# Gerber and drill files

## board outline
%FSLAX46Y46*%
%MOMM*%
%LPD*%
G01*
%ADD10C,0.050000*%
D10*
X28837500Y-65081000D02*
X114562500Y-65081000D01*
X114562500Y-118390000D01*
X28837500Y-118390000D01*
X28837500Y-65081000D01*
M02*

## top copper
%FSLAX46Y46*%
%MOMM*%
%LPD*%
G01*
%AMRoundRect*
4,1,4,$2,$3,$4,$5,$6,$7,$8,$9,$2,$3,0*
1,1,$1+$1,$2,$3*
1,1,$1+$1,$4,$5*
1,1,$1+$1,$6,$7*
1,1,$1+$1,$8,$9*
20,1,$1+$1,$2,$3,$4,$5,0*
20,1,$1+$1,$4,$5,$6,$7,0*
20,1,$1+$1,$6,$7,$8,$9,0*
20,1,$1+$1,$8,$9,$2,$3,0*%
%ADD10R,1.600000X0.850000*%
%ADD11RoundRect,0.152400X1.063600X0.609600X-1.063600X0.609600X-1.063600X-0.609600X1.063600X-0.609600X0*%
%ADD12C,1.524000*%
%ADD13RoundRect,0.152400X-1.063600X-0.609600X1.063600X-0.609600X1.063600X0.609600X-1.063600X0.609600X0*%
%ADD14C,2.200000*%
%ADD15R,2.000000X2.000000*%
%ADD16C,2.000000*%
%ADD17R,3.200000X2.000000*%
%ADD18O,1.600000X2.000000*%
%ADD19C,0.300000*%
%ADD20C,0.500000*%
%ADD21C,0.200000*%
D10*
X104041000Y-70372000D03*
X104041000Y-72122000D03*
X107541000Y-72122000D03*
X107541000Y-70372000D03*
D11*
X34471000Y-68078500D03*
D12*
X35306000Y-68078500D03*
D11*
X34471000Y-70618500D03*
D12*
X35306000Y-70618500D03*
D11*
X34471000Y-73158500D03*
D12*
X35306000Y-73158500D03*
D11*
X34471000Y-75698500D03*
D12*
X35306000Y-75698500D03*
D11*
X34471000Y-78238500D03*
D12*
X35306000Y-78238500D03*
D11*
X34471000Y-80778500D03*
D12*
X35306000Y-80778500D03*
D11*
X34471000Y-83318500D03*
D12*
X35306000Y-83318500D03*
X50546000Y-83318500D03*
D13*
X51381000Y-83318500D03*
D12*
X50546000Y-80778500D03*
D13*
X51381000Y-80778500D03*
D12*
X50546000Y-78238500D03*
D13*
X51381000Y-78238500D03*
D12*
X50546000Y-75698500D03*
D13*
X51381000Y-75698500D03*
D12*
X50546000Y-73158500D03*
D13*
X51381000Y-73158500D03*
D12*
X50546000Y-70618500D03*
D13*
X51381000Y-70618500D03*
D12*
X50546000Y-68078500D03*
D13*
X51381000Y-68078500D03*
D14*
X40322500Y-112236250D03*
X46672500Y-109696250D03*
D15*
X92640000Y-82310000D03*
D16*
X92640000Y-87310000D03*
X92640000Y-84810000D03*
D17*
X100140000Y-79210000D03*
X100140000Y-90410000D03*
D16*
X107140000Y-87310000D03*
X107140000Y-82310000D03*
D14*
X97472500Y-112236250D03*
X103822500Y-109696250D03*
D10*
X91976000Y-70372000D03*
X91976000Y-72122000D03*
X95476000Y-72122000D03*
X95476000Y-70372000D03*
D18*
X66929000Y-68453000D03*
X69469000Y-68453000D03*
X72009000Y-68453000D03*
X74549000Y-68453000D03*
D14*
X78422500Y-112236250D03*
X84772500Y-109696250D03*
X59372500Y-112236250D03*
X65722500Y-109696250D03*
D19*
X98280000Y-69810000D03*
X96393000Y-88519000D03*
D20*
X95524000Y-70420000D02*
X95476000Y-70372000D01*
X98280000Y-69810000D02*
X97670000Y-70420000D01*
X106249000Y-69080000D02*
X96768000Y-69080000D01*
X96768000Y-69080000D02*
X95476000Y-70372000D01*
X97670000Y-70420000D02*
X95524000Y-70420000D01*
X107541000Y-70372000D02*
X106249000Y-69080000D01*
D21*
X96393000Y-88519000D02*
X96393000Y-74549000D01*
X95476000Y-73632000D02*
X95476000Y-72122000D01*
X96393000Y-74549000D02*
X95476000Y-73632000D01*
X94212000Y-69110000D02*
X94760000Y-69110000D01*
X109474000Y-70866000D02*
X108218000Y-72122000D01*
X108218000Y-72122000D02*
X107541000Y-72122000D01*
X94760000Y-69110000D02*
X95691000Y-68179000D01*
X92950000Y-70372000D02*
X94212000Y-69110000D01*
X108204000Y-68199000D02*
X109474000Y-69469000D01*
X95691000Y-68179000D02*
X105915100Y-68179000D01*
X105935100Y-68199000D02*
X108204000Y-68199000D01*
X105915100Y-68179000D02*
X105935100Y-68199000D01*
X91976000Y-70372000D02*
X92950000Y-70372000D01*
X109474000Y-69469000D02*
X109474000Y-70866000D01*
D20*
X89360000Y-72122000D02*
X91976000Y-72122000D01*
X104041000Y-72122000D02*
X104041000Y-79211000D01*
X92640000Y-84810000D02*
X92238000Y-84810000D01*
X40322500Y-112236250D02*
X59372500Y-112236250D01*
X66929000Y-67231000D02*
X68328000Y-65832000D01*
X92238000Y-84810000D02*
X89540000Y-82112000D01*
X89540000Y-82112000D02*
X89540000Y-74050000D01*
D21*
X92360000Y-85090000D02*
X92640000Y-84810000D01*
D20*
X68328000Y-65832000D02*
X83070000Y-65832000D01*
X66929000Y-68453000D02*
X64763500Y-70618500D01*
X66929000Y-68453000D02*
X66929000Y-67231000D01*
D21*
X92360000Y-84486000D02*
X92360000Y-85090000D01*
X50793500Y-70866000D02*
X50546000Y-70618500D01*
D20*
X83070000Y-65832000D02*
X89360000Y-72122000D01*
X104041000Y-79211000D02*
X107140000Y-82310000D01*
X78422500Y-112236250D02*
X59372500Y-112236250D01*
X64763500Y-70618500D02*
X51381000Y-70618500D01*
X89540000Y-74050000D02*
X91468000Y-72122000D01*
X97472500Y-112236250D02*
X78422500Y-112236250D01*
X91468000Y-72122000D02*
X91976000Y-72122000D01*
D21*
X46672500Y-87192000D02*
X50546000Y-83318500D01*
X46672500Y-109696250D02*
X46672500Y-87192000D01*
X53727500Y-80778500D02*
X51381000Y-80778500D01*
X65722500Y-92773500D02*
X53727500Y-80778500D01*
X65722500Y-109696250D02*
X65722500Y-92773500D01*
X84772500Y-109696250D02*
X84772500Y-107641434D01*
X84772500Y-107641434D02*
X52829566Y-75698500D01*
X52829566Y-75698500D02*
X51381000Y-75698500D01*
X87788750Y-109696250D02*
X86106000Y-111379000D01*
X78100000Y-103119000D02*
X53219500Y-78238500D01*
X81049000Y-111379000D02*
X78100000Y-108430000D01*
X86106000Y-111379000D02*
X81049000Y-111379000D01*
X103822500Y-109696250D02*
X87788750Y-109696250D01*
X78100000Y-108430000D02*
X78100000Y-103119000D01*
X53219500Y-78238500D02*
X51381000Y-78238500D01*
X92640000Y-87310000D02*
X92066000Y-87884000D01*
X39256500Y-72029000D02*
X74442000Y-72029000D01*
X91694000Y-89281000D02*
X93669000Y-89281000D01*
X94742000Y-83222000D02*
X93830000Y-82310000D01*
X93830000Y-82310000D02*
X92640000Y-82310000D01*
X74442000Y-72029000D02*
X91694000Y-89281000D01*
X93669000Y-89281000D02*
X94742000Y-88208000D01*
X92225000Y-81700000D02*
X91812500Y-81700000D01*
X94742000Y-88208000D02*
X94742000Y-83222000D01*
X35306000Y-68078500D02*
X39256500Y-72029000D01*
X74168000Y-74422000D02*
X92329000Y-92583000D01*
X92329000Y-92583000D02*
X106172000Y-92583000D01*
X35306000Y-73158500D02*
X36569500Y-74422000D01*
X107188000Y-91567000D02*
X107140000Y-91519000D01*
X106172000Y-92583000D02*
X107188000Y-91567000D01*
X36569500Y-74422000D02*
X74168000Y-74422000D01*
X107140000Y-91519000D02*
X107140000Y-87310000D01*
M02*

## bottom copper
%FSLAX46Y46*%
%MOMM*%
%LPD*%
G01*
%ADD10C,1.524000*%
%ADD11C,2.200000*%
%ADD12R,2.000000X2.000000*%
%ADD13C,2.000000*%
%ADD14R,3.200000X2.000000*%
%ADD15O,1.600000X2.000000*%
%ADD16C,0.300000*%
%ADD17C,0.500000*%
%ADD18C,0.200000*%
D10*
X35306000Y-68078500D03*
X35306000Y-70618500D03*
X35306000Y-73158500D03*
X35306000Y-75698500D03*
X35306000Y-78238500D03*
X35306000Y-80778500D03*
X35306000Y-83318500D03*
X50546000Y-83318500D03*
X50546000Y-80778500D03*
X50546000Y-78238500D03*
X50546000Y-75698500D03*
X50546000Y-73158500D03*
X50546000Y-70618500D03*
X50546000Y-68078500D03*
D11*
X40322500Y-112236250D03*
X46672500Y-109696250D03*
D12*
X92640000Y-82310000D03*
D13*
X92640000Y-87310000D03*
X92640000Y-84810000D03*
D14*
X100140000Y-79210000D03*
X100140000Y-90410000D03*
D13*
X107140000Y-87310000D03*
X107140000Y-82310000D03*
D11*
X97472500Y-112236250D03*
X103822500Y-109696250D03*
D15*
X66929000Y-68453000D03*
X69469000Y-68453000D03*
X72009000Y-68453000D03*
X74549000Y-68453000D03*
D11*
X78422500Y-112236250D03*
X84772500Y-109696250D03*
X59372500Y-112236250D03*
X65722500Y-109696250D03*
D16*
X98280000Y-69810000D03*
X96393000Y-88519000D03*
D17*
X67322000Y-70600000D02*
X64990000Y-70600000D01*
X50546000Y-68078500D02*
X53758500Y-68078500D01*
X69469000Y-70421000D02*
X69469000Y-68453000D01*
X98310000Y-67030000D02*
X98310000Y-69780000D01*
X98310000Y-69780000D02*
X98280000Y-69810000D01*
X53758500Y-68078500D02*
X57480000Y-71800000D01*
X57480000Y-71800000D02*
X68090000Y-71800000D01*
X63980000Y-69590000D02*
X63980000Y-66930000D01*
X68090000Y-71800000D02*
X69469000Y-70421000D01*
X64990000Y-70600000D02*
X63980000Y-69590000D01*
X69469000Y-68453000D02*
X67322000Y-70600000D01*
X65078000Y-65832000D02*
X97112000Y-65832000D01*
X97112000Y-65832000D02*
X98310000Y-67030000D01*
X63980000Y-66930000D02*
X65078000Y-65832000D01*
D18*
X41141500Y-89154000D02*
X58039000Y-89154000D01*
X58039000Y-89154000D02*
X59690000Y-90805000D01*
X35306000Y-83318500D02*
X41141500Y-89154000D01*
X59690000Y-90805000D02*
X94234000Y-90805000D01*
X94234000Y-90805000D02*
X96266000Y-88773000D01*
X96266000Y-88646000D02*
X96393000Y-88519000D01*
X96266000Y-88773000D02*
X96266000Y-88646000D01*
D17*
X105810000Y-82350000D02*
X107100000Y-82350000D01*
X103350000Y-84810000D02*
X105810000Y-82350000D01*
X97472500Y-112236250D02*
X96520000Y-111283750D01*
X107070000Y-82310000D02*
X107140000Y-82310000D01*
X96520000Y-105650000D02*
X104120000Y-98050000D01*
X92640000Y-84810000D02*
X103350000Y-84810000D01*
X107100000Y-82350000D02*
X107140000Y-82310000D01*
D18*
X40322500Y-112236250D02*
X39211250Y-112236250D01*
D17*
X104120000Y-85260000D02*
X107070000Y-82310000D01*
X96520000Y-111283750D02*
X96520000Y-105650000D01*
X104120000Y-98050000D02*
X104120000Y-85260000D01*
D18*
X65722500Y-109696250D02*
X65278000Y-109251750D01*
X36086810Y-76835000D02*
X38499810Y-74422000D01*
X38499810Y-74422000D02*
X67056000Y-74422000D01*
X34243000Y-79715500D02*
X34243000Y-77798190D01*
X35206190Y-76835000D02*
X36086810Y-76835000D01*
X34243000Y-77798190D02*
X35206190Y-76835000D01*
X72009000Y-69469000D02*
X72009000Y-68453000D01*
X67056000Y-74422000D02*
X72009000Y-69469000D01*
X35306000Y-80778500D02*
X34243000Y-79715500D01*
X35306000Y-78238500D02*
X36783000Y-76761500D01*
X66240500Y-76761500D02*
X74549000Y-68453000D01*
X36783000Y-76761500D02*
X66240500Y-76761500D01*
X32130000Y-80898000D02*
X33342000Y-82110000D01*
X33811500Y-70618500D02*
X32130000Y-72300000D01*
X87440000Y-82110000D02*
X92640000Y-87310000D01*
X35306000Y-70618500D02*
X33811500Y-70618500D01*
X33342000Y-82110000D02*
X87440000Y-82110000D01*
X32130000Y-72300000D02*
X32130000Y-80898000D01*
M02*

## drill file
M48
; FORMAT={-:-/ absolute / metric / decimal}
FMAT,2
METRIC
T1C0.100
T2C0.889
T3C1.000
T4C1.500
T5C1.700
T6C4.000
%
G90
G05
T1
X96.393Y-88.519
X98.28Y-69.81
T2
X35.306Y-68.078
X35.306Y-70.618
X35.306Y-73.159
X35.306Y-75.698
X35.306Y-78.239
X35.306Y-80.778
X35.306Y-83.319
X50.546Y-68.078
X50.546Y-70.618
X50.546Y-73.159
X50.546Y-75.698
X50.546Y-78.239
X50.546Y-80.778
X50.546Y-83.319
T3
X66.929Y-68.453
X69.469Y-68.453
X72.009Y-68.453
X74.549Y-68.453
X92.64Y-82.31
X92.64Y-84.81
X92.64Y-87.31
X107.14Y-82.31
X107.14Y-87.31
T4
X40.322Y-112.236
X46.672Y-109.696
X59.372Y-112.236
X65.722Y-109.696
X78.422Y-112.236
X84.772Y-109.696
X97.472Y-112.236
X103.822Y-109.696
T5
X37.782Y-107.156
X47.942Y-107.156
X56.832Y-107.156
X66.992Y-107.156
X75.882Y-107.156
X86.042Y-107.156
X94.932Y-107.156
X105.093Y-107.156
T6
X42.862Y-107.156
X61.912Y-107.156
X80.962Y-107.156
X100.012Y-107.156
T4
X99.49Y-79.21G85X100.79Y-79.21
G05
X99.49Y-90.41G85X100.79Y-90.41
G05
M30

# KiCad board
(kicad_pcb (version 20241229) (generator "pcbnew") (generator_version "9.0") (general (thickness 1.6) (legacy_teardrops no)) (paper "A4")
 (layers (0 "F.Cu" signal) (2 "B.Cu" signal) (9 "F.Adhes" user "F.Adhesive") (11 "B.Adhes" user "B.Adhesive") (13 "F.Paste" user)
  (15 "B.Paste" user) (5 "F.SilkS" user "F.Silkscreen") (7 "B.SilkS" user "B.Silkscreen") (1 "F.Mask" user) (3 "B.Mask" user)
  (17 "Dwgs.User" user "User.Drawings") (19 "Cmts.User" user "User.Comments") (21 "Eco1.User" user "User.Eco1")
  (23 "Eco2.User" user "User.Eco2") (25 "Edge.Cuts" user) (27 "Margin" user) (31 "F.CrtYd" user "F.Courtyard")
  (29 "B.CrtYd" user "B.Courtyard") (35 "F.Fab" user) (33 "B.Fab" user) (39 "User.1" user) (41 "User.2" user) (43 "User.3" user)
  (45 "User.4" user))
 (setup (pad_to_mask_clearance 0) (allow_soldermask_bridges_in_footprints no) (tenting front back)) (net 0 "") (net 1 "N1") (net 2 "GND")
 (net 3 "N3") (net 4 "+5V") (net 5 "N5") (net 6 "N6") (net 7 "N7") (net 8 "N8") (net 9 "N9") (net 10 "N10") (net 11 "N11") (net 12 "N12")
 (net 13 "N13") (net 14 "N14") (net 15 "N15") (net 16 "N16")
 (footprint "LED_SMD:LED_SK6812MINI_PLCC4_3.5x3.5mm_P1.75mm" (layer "F.Cu") (at 105.791 71.247)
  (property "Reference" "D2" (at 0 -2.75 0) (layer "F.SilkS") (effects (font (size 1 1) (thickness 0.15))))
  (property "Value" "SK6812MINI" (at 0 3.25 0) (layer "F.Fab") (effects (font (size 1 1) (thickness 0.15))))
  (pad "1" smd rect (at -1.75 -0.875) (size 1.6 0.85) (layers "F.Cu" "F.Mask" "F.Paste") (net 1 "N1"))
  (pad "2" smd rect (at -1.75 0.875) (size 1.6 0.85) (layers "F.Cu" "F.Mask" "F.Paste") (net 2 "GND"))
  (pad "3" smd rect (at 1.75 0.875) (size 1.6 0.85) (layers "F.Cu" "F.Mask" "F.Paste") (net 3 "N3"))
  (pad "4" smd rect (at 1.75 -0.875) (size 1.6 0.85) (layers "F.Cu" "F.Mask" "F.Paste") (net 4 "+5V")))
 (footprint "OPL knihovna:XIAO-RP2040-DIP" (layer "F.Cu") (at 42.926 75.6985)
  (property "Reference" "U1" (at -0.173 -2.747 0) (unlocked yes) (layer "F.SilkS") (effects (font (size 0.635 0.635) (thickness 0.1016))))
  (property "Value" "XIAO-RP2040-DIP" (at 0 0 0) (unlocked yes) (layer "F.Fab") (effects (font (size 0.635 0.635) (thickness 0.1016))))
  (pad "1" smd roundrect (at -8.455 -7.62 180) (size 2.432 1.524) (layers "F.Cu" "F.Mask") (roundrect_rratio 0.1) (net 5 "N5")
   (thermal_bridge_angle 45))
  (pad "1" thru_hole circle (at -7.62 -7.62 180) (size 1.524 1.524) (drill 0.889) (layers "*.Cu" "*.Mask") (remove_unused_layers no)
   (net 5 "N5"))
  (pad "2" smd roundrect (at -8.455 -5.08 180) (size 2.432 1.524) (layers "F.Cu" "F.Mask") (roundrect_rratio 0.1) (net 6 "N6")
   (thermal_bridge_angle 45))
  (pad "2" thru_hole circle (at -7.62 -5.08 180) (size 1.524 1.524) (drill 0.889) (layers "*.Cu" "*.Mask") (remove_unused_layers no)
   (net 6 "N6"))
  (pad "3" smd roundrect (at -8.455 -2.54 180) (size 2.432 1.524) (layers "F.Cu" "F.Mask") (roundrect_rratio 0.1) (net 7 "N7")
   (thermal_bridge_angle 45))
  (pad "3" thru_hole circle (at -7.62 -2.54 180) (size 1.524 1.524) (drill 0.889) (layers "*.Cu" "*.Mask") (remove_unused_layers no)
   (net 7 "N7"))
  (pad "4" smd roundrect (at -8.455 0 180) (size 2.432 1.524) (layers "F.Cu" "F.Mask") (roundrect_rratio 0.1) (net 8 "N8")
   (thermal_bridge_angle 45))
  (pad "4" thru_hole circle (at -7.62 0 180) (size 1.524 1.524) (drill 0.889) (layers "*.Cu" "*.Mask") (remove_unused_layers no)
   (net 8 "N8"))
  (pad "5" smd roundrect (at -8.455 2.54 180) (size 2.432 1.524) (layers "F.Cu" "F.Mask") (roundrect_rratio 0.1) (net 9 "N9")
   (thermal_bridge_angle 45))
  (pad "5" thru_hole circle (at -7.62 2.54 180) (size 1.524 1.524) (drill 0.889) (layers "*.Cu" "*.Mask") (remove_unused_layers no)
   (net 9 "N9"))
  (pad "6" smd roundrect (at -8.455 5.08 180) (size 2.432 1.524) (layers "F.Cu" "F.Mask") (roundrect_rratio 0.1) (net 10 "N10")
   (thermal_bridge_angle 45))
  (pad "6" thru_hole circle (at -7.62 5.08 180) (size 1.524 1.524) (drill 0.889) (layers "*.Cu" "*.Mask") (remove_unused_layers no)
   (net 10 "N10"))
  (pad "7" smd roundrect (at -8.455 7.62 180) (size 2.432 1.524) (layers "F.Cu" "F.Mask") (roundrect_rratio 0.1) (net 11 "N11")
   (thermal_bridge_angle 45))
  (pad "7" thru_hole circle (at -7.62 7.62 180) (size 1.524 1.524) (drill 0.889) (layers "*.Cu" "*.Mask") (remove_unused_layers no)
   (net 11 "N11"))
  (pad "8" thru_hole circle (at 7.62 7.62) (size 1.524 1.524) (drill 0.889) (layers "*.Cu" "*.Mask") (remove_unused_layers no)
   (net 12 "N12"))
  (pad "8" smd roundrect (at 8.455 7.62) (size 2.432 1.524) (layers "F.Cu" "F.Mask") (roundrect_rratio 0.1) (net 12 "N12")
   (thermal_bridge_angle 45))
  (pad "9" thru_hole circle (at 7.62 5.08) (size 1.524 1.524) (drill 0.889) (layers "*.Cu" "*.Mask") (remove_unused_layers no)
   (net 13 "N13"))
  (pad "9" smd roundrect (at 8.455 5.08) (size 2.432 1.524) (layers "F.Cu" "F.Mask") (roundrect_rratio 0.1) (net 13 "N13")
   (thermal_bridge_angle 45))
  (pad "10" thru_hole circle (at 7.62 2.54) (size 1.524 1.524) (drill 0.889) (layers "*.Cu" "*.Mask") (remove_unused_layers no)
   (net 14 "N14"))
  (pad "10" smd roundrect (at 8.455 2.54) (size 2.432 1.524) (layers "F.Cu" "F.Mask") (roundrect_rratio 0.1) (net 14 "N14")
   (thermal_bridge_angle 45))
  (pad "11" thru_hole circle (at 7.62 0) (size 1.524 1.524) (drill 0.889) (layers "*.Cu" "*.Mask") (remove_unused_layers no) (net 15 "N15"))
  (pad "11" smd roundrect (at 8.455 0) (size 2.432 1.524) (layers "F.Cu" "F.Mask") (roundrect_rratio 0.1) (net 15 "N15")
   (thermal_bridge_angle 45))
  (pad "12" thru_hole circle (at 7.62 -2.54) (size 1.524 1.524) (drill 0.889) (layers "*.Cu" "*.Mask") (remove_unused_layers no)
   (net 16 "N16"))
  (pad "12" smd roundrect (at 8.455 -2.54) (size 2.432 1.524) (layers "F.Cu" "F.Mask") (roundrect_rratio 0.1) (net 16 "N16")
   (thermal_bridge_angle 45))
  (pad "13" thru_hole circle (at 7.62 -5.08) (size 1.524 1.524) (drill 0.889) (layers "*.Cu" "*.Mask") (remove_unused_layers no)
   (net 2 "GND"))
  (pad "13" smd roundrect (at 8.455 -5.08) (size 2.432 1.524) (layers "F.Cu" "F.Mask") (roundrect_rratio 0.1) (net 2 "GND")
   (thermal_bridge_angle 45))
  (pad "14" thru_hole circle (at 7.62 -7.62) (size 1.524 1.524) (drill 0.889) (layers "*.Cu" "*.Mask") (remove_unused_layers no)
   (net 4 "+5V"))
  (pad "14" smd roundrect (at 8.455 -7.62) (size 2.432 1.524) (layers "F.Cu" "F.Mask") (roundrect_rratio 0.1) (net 4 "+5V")
   (thermal_bridge_angle 45)))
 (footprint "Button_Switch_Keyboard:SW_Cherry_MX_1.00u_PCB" (layer "F.Cu") (at 40.3225 112.23625 180)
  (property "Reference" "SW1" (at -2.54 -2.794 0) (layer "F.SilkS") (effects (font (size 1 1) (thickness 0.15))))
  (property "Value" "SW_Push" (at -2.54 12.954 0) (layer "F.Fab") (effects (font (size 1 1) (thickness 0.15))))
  (pad "" np_thru_hole circle (at -7.62 5.08 180) (size 1.7 1.7) (drill 1.7) (layers "*.Cu" "*.Mask"))
  (pad "" np_thru_hole circle (at -2.54 5.08 180) (size 4 4) (drill 4) (layers "*.Cu" "*.Mask"))
  (pad "" np_thru_hole circle (at 2.54 5.08 180) (size 1.7 1.7) (drill 1.7) (layers "*.Cu" "*.Mask"))
  (pad "1" thru_hole circle (at 0 0 180) (size 2.2 2.2) (drill 1.5) (layers "*.Cu" "*.Mask") (remove_unused_layers no) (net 2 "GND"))
  (pad "2" thru_hole circle (at -6.35 2.54 180) (size 2.2 2.2) (drill 1.5) (layers "*.Cu" "*.Mask") (remove_unused_layers no) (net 12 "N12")))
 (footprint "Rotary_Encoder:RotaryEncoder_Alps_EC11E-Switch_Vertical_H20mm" (layer "F.Cu") (at 92.64 82.31)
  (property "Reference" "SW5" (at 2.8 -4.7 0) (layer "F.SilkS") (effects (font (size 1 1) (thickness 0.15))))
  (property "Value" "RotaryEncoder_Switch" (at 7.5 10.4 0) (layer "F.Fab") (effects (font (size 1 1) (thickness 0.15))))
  (pad "A" thru_hole rect (at 0 0) (size 2 2) (drill 1) (layers "*.Cu" "*.Mask") (remove_unused_layers no) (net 5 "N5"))
  (pad "B" thru_hole circle (at 0 5) (size 2 2) (drill 1) (layers "*.Cu" "*.Mask") (remove_unused_layers no) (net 6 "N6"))
  (pad "C" thru_hole circle (at 0 2.5) (size 2 2) (drill 1) (layers "*.Cu" "*.Mask") (remove_unused_layers no) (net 2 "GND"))
  (pad "MP" thru_hole rect (at 7.5 -3.1) (size 3.2 2) (drill oval 2.8 1.5) (layers "*.Cu" "*.Mask") (remove_unused_layers no))
  (pad "MP" thru_hole rect (at 7.5 8.1) (size 3.2 2) (drill oval 2.8 1.5) (layers "*.Cu" "*.Mask") (remove_unused_layers no))
  (pad "S1" thru_hole circle (at 14.5 5) (size 2 2) (drill 1) (layers "*.Cu" "*.Mask") (remove_unused_layers no) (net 7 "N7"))
  (pad "S2" thru_hole circle (at 14.5 0) (size 2 2) (drill 1) (layers "*.Cu" "*.Mask") (remove_unused_layers no) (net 2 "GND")))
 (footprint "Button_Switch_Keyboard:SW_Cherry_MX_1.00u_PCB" (layer "F.Cu") (at 97.4725 112.23625 180)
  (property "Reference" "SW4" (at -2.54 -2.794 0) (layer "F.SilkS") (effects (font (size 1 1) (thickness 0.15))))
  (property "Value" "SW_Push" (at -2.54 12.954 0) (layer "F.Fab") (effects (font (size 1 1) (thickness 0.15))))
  (pad "" np_thru_hole circle (at -7.62 5.08 180) (size 1.7 1.7) (drill 1.7) (layers "*.Cu" "*.Mask"))
  (pad "" np_thru_hole circle (at -2.54 5.08 180) (size 4 4) (drill 4) (layers "*.Cu" "*.Mask"))
  (pad "" np_thru_hole circle (at 2.54 5.08 180) (size 1.7 1.7) (drill 1.7) (layers "*.Cu" "*.Mask"))
  (pad "1" thru_hole circle (at 0 0 180) (size 2.2 2.2) (drill 1.5) (layers "*.Cu" "*.Mask") (remove_unused_layers no) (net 2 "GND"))
  (pad "2" thru_hole circle (at -6.35 2.54 180) (size 2.2 2.2) (drill 1.5) (layers "*.Cu" "*.Mask") (remove_unused_layers no) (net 14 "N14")))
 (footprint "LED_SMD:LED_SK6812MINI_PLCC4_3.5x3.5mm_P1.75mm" (layer "F.Cu") (at 93.726 71.247)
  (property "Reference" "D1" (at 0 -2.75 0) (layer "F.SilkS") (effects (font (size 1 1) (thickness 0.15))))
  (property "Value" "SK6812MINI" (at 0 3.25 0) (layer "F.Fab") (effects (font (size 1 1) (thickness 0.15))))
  (pad "1" smd rect (at -1.75 -0.875) (size 1.6 0.85) (layers "F.Cu" "F.Mask" "F.Paste") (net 3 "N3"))
  (pad "2" smd rect (at -1.75 0.875) (size 1.6 0.85) (layers "F.Cu" "F.Mask" "F.Paste") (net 2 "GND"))
  (pad "3" smd rect (at 1.75 0.875) (size 1.6 0.85) (layers "F.Cu" "F.Mask" "F.Paste") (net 11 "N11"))
  (pad "4" smd rect (at 1.75 -0.875) (size 1.6 0.85) (layers "F.Cu" "F.Mask" "F.Paste") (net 4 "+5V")))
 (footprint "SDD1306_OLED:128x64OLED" (layer "F.Cu") (at 70.549 79.053)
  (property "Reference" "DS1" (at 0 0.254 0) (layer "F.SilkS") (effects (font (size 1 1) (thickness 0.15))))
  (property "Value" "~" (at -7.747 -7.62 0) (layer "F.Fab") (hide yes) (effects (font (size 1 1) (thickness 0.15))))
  (pad "1" thru_hole oval (at -3.62 -10.6 90) (size 2 1.6) (drill 1) (layers "*.Cu" "*.Mask") (remove_unused_layers no) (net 2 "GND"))
  (pad "2" thru_hole oval (at -1.08 -10.6 90) (size 2 1.6) (drill 1) (layers "*.Cu" "*.Mask") (remove_unused_layers no) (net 4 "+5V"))
  (pad "3" thru_hole oval (at 1.46 -10.6 90) (size 2 1.6) (drill 1) (layers "*.Cu" "*.Mask") (remove_unused_layers no) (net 10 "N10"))
  (pad "4" thru_hole oval (at 4 -10.6 90) (size 2 1.6) (drill 1) (layers "*.Cu" "*.Mask") (remove_unused_layers no) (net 9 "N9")))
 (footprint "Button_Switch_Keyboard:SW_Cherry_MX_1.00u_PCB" (layer "F.Cu") (at 78.4225 112.23625 180)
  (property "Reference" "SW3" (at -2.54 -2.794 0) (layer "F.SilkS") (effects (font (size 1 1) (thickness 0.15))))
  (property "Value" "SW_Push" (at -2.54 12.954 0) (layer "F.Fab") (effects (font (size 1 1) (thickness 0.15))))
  (pad "" np_thru_hole circle (at -7.62 5.08 180) (size 1.7 1.7) (drill 1.7) (layers "*.Cu" "*.Mask"))
  (pad "" np_thru_hole circle (at -2.54 5.08 180) (size 4 4) (drill 4) (layers "*.Cu" "*.Mask"))
  (pad "" np_thru_hole circle (at 2.54 5.08 180) (size 1.7 1.7) (drill 1.7) (layers "*.Cu" "*.Mask"))
  (pad "1" thru_hole circle (at 0 0 180) (size 2.2 2.2) (drill 1.5) (layers "*.Cu" "*.Mask") (remove_unused_layers no) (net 2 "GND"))
  (pad "2" thru_hole circle (at -6.35 2.54 180) (size 2.2 2.2) (drill 1.5) (layers "*.Cu" "*.Mask") (remove_unused_layers no) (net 15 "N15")))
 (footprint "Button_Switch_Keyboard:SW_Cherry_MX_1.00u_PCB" (layer "F.Cu") (at 59.3725 112.23625 180)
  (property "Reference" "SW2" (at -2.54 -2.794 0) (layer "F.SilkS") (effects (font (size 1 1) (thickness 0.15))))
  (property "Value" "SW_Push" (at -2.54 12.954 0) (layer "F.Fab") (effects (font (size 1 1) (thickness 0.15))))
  (pad "" np_thru_hole circle (at -7.62 5.08 180) (size 1.7 1.7) (drill 1.7) (layers "*.Cu" "*.Mask"))
  (pad "" np_thru_hole circle (at -2.54 5.08 180) (size 4 4) (drill 4) (layers "*.Cu" "*.Mask"))
  (pad "" np_thru_hole circle (at 2.54 5.08 180) (size 1.7 1.7) (drill 1.7) (layers "*.Cu" "*.Mask"))
  (pad "1" thru_hole circle (at 0 0 180) (size 2.2 2.2) (drill 1.5) (layers "*.Cu" "*.Mask") (remove_unused_layers no) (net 2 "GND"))
  (pad "2" thru_hole circle (at -6.35 2.54 180) (size 2.2 2.2) (drill 1.5) (layers "*.Cu" "*.Mask") (remove_unused_layers no) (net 13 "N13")))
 (gr_rect (start 28.8375 65.081) (end 114.5625 118.39) (stroke (width 0.05) (type default)) (fill no) (layer "Edge.Cuts"))
 (segment (start 95.524 70.42) (end 95.476 70.372) (width 0.5) (layer "F.Cu") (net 4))
 (segment (start 98.28 69.81) (end 97.67 70.42) (width 0.5) (layer "F.Cu") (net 4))
 (segment (start 106.249 69.08) (end 96.768 69.08) (width 0.5) (layer "F.Cu") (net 4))
 (segment (start 96.768 69.08) (end 95.476 70.372) (width 0.5) (layer "F.Cu") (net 4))
 (segment (start 97.67 70.42) (end 95.524 70.42) (width 0.5) (layer "F.Cu") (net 4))
 (segment (start 107.541 70.372) (end 106.249 69.08) (width 0.5) (layer "F.Cu") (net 4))
 (via micro (at 98.28 69.81) (size 0.3) (drill 0.1) (layers "F.Cu" "B.Cu") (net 4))
 (segment (start 67.322 70.6) (end 64.99 70.6) (width 0.5) (layer "B.Cu") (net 4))
 (segment (start 50.546 68.0785) (end 53.7585 68.0785) (width 0.5) (layer "B.Cu") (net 4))
 (segment (start 69.469 70.421) (end 69.469 68.453) (width 0.5) (layer "B.Cu") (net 4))
 (segment (start 98.31 67.03) (end 98.31 69.78) (width 0.5) (layer "B.Cu") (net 4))
 (segment (start 98.31 69.78) (end 98.28 69.81) (width 0.5) (layer "B.Cu") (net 4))
 (segment (start 53.7585 68.0785) (end 57.48 71.8) (width 0.5) (layer "B.Cu") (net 4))
 (segment (start 57.48 71.8) (end 68.09 71.8) (width 0.5) (layer "B.Cu") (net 4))
 (segment (start 63.98 69.59) (end 63.98 66.93) (width 0.5) (layer "B.Cu") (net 4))
 (segment (start 68.09 71.8) (end 69.469 70.421) (width 0.5) (layer "B.Cu") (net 4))
 (segment (start 64.99 70.6) (end 63.98 69.59) (width 0.5) (layer "B.Cu") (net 4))
 (segment (start 69.469 68.453) (end 67.322 70.6) (width 0.5) (layer "B.Cu") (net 4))
 (segment (start 65.078 65.832) (end 97.112 65.832) (width 0.5) (layer "B.Cu") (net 4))
 (segment (start 97.112 65.832) (end 98.31 67.03) (width 0.5) (layer "B.Cu") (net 4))
 (segment (start 63.98 66.93) (end 65.078 65.832) (width 0.5) (layer "B.Cu") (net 4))
 (segment (start 96.393 88.519) (end 96.393 74.549) (width 0.2) (layer "F.Cu") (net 11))
 (segment (start 95.476 73.632) (end 95.476 72.122) (width 0.2) (layer "F.Cu") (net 11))
 (segment (start 96.393 74.549) (end 95.476 73.632) (width 0.2) (layer "F.Cu") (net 11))
 (via micro (at 96.393 88.519) (size 0.3) (drill 0.1) (layers "F.Cu" "B.Cu") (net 11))
 (segment (start 41.1415 89.154) (end 58.039 89.154) (width 0.2) (layer "B.Cu") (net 11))
 (segment (start 58.039 89.154) (end 59.69 90.805) (width 0.2) (layer "B.Cu") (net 11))
 (segment (start 35.306 83.3185) (end 41.1415 89.154) (width 0.2) (layer "B.Cu") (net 11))
 (segment (start 59.69 90.805) (end 94.234 90.805) (width 0.2) (layer "B.Cu") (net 11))
 (segment (start 94.234 90.805) (end 96.266 88.773) (width 0.2) (layer "B.Cu") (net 11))
 (segment (start 96.266 88.646) (end 96.393 88.519) (width 0.2) (layer "B.Cu") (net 11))
 (segment (start 96.266 88.773) (end 96.266 88.646) (width 0.2) (layer "B.Cu") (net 11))
 (segment (start 94.212 69.11) (end 94.76 69.11) (width 0.2) (layer "F.Cu") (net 3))
 (segment (start 109.474 70.866) (end 108.218 72.122) (width 0.2) (layer "F.Cu") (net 3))
 (segment (start 108.218 72.122) (end 107.541 72.122) (width 0.2) (layer "F.Cu") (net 3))
 (segment (start 94.76 69.11) (end 95.691 68.179) (width 0.2) (layer "F.Cu") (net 3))
 (segment (start 92.95 70.372) (end 94.212 69.11) (width 0.2) (layer "F.Cu") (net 3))
 (segment (start 108.204 68.199) (end 109.474 69.469) (width 0.2) (layer "F.Cu") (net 3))
 (segment (start 95.691 68.179) (end 105.9151 68.179) (width 0.2) (layer "F.Cu") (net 3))
 (segment (start 105.9351 68.199) (end 108.204 68.199) (width 0.2) (layer "F.Cu") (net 3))
 (segment (start 105.9151 68.179) (end 105.9351 68.199) (width 0.2) (layer "F.Cu") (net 3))
 (segment (start 91.976 70.372) (end 92.95 70.372) (width 0.2) (layer "F.Cu") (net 3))
 (segment (start 109.474 69.469) (end 109.474 70.866) (width 0.2) (layer "F.Cu") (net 3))
 (segment (start 89.36 72.122) (end 91.976 72.122) (width 0.5) (layer "F.Cu") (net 2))
 (segment (start 104.041 72.122) (end 104.041 79.211) (width 0.5) (layer "F.Cu") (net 2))
 (segment (start 92.64 84.81) (end 92.238 84.81) (width 0.5) (layer "F.Cu") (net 2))
 (segment (start 40.3225 112.23625) (end 59.3725 112.23625) (width 0.5) (layer "F.Cu") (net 2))
 (segment (start 66.929 67.231) (end 68.328 65.832) (width 0.5) (layer "F.Cu") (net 2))
 (segment (start 92.238 84.81) (end 89.54 82.112) (width 0.5) (layer "F.Cu") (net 2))
 (segment (start 89.54 82.112) (end 89.54 74.05) (width 0.5) (layer "F.Cu") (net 2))
 (segment (start 92.36 85.09) (end 92.64 84.81) (width 0.2) (layer "F.Cu") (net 2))
 (segment (start 68.328 65.832) (end 83.07 65.832) (width 0.5) (layer "F.Cu") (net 2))
 (segment (start 66.929 68.453) (end 64.7635 70.6185) (width 0.5) (layer "F.Cu") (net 2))
 (segment (start 66.929 68.453) (end 66.929 67.231) (width 0.5) (layer "F.Cu") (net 2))
 (segment (start 92.36 84.486) (end 92.36 85.09) (width 0.2) (layer "F.Cu") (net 2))
 (segment (start 50.7935 70.866) (end 50.546 70.6185) (width 0.2) (layer "F.Cu") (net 2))
 (segment (start 83.07 65.832) (end 89.36 72.122) (width 0.5) (layer "F.Cu") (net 2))
 (segment (start 104.041 79.211) (end 107.14 82.31) (width 0.5) (layer "F.Cu") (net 2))
 (segment (start 78.4225 112.23625) (end 59.3725 112.23625) (width 0.5) (layer "F.Cu") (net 2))
 (segment (start 64.7635 70.6185) (end 51.381 70.6185) (width 0.5) (layer "F.Cu") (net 2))
 (segment (start 89.54 74.05) (end 91.468 72.122) (width 0.5) (layer "F.Cu") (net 2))
 (segment (start 97.4725 112.23625) (end 78.4225 112.23625) (width 0.5) (layer "F.Cu") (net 2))
 (segment (start 91.468 72.122) (end 91.976 72.122) (width 0.5) (layer "F.Cu") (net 2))
 (segment (start 105.81 82.35) (end 107.1 82.35) (width 0.5) (layer "B.Cu") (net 2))
 (segment (start 103.35 84.81) (end 105.81 82.35) (width 0.5) (layer "B.Cu") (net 2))
 (segment (start 97.4725 112.23625) (end 96.52 111.28375) (width 0.5) (layer "B.Cu") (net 2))
 (segment (start 107.07 82.31) (end 107.14 82.31) (width 0.5) (layer "B.Cu") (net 2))
 (segment (start 96.52 105.65) (end 104.12 98.05) (width 0.5) (layer "B.Cu") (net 2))
 (segment (start 92.64 84.81) (end 103.35 84.81) (width 0.5) (layer "B.Cu") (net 2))
 (segment (start 107.1 82.35) (end 107.14 82.31) (width 0.5) (layer "B.Cu") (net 2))
 (segment (start 40.3225 112.23625) (end 39.21125 112.23625) (width 0.2) (layer "B.Cu") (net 2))
 (segment (start 104.12 85.26) (end 107.07 82.31) (width 0.5) (layer "B.Cu") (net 2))
 (segment (start 96.52 111.28375) (end 96.52 105.65) (width 0.5) (layer "B.Cu") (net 2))
 (segment (start 104.12 98.05) (end 104.12 85.26) (width 0.5) (layer "B.Cu") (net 2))
 (segment (start 46.6725 87.192) (end 50.546 83.3185) (width 0.2) (layer "F.Cu") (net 12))
 (segment (start 46.6725 109.69625) (end 46.6725 87.192) (width 0.2) (layer "F.Cu") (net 12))
 (segment (start 53.7275 80.7785) (end 51.381 80.7785) (width 0.2) (layer "F.Cu") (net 13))
 (segment (start 65.7225 92.7735) (end 53.7275 80.7785) (width 0.2) (layer "F.Cu") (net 13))
 (segment (start 65.7225 109.69625) (end 65.7225 92.7735) (width 0.2) (layer "F.Cu") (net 13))
 (segment (start 65.7225 109.69625) (end 65.278 109.25175) (width 0.2) (layer "B.Cu") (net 13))
 (segment (start 84.7725 109.69625) (end 84.7725 107.641434) (width 0.2) (layer "F.Cu") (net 15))
 (segment (start 84.7725 107.641434) (end 52.829566 75.6985) (width 0.2) (layer "F.Cu") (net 15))
 (segment (start 52.829566 75.6985) (end 51.381 75.6985) (width 0.2) (layer "F.Cu") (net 15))
 (segment (start 87.78875 109.69625) (end 86.106 111.379) (width 0.2) (layer "F.Cu") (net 14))
 (segment (start 78.1 103.119) (end 53.2195 78.2385) (width 0.2) (layer "F.Cu") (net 14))
 (segment (start 81.049 111.379) (end 78.1 108.43) (width 0.2) (layer "F.Cu") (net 14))
 (segment (start 86.106 111.379) (end 81.049 111.379) (width 0.2) (layer "F.Cu") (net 14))
 (segment (start 103.8225 109.69625) (end 87.78875 109.69625) (width 0.2) (layer "F.Cu") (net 14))
 (segment (start 78.1 108.43) (end 78.1 103.119) (width 0.2) (layer "F.Cu") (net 14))
 (segment (start 53.2195 78.2385) (end 51.381 78.2385) (width 0.2) (layer "F.Cu") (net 14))
 (segment (start 36.08681 76.835) (end 38.49981 74.422) (width 0.2) (layer "B.Cu") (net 10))
 (segment (start 38.49981 74.422) (end 67.056 74.422) (width 0.2) (layer "B.Cu") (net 10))
 (segment (start 34.243 79.7155) (end 34.243 77.79819) (width 0.2) (layer "B.Cu") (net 10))
 (segment (start 35.20619 76.835) (end 36.08681 76.835) (width 0.2) (layer "B.Cu") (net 10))
 (segment (start 34.243 77.79819) (end 35.20619 76.835) (width 0.2) (layer "B.Cu") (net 10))
 (segment (start 72.009 69.469) (end 72.009 68.453) (width 0.2) (layer "B.Cu") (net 10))
 (segment (start 67.056 74.422) (end 72.009 69.469) (width 0.2) (layer "B.Cu") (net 10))
 (segment (start 35.306 80.7785) (end 34.243 79.7155) (width 0.2) (layer "B.Cu") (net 10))
 (segment (start 35.306 78.2385) (end 36.783 76.7615) (width 0.2) (layer "B.Cu") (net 9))
 (segment (start 66.2405 76.7615) (end 74.549 68.453) (width 0.2) (layer "B.Cu") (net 9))
 (segment (start 36.783 76.7615) (end 66.2405 76.7615) (width 0.2) (layer "B.Cu") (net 9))
 (segment (start 92.64 87.31) (end 92.066 87.884) (width 0.2) (layer "F.Cu") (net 6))
 (segment (start 32.13 80.898) (end 33.342 82.11) (width 0.2) (layer "B.Cu") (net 6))
 (segment (start 33.8115 70.6185) (end 32.13 72.3) (width 0.2) (layer "B.Cu") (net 6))
 (segment (start 87.44 82.11) (end 92.64 87.31) (width 0.2) (layer "B.Cu") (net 6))
 (segment (start 35.306 70.6185) (end 33.8115 70.6185) (width 0.2) (layer "B.Cu") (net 6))
 (segment (start 33.342 82.11) (end 87.44 82.11) (width 0.2) (layer "B.Cu") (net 6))
 (segment (start 32.13 72.3) (end 32.13 80.898) (width 0.2) (layer "B.Cu") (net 6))
 (segment (start 39.2565 72.029) (end 74.442 72.029) (width 0.2) (layer "F.Cu") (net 5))
 (segment (start 91.694 89.281) (end 93.669 89.281) (width 0.2) (layer "F.Cu") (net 5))
 (segment (start 94.742 83.222) (end 93.83 82.31) (width 0.2) (layer "F.Cu") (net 5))
 (segment (start 93.83 82.31) (end 92.64 82.31) (width 0.2) (layer "F.Cu") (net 5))
 (segment (start 74.442 72.029) (end 91.694 89.281) (width 0.2) (layer "F.Cu") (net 5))
 (segment (start 93.669 89.281) (end 94.742 88.208) (width 0.2) (layer "F.Cu") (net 5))
 (segment (start 92.225 81.7) (end 91.8125 81.7) (width 0.2) (layer "F.Cu") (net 5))
 (segment (start 94.742 88.208) (end 94.742 83.222) (width 0.2) (layer "F.Cu") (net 5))
 (segment (start 35.306 68.0785) (end 39.2565 72.029) (width 0.2) (layer "F.Cu") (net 5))
 (segment (start 74.168 74.422) (end 92.329 92.583) (width 0.2) (layer "F.Cu") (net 7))
 (segment (start 92.329 92.583) (end 106.172 92.583) (width 0.2) (layer "F.Cu") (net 7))
 (segment (start 35.306 73.1585) (end 36.5695 74.422) (width 0.2) (layer "F.Cu") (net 7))
 (segment (start 107.188 91.567) (end 107.14 91.519) (width 0.2) (layer "F.Cu") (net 7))
 (segment (start 106.172 92.583) (end 107.188 91.567) (width 0.2) (layer "F.Cu") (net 7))
 (segment (start 36.5695 74.422) (end 74.168 74.422) (width 0.2) (layer "F.Cu") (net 7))
 (segment (start 107.14 91.519) (end 107.14 87.31) (width 0.2) (layer "F.Cu") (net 7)))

